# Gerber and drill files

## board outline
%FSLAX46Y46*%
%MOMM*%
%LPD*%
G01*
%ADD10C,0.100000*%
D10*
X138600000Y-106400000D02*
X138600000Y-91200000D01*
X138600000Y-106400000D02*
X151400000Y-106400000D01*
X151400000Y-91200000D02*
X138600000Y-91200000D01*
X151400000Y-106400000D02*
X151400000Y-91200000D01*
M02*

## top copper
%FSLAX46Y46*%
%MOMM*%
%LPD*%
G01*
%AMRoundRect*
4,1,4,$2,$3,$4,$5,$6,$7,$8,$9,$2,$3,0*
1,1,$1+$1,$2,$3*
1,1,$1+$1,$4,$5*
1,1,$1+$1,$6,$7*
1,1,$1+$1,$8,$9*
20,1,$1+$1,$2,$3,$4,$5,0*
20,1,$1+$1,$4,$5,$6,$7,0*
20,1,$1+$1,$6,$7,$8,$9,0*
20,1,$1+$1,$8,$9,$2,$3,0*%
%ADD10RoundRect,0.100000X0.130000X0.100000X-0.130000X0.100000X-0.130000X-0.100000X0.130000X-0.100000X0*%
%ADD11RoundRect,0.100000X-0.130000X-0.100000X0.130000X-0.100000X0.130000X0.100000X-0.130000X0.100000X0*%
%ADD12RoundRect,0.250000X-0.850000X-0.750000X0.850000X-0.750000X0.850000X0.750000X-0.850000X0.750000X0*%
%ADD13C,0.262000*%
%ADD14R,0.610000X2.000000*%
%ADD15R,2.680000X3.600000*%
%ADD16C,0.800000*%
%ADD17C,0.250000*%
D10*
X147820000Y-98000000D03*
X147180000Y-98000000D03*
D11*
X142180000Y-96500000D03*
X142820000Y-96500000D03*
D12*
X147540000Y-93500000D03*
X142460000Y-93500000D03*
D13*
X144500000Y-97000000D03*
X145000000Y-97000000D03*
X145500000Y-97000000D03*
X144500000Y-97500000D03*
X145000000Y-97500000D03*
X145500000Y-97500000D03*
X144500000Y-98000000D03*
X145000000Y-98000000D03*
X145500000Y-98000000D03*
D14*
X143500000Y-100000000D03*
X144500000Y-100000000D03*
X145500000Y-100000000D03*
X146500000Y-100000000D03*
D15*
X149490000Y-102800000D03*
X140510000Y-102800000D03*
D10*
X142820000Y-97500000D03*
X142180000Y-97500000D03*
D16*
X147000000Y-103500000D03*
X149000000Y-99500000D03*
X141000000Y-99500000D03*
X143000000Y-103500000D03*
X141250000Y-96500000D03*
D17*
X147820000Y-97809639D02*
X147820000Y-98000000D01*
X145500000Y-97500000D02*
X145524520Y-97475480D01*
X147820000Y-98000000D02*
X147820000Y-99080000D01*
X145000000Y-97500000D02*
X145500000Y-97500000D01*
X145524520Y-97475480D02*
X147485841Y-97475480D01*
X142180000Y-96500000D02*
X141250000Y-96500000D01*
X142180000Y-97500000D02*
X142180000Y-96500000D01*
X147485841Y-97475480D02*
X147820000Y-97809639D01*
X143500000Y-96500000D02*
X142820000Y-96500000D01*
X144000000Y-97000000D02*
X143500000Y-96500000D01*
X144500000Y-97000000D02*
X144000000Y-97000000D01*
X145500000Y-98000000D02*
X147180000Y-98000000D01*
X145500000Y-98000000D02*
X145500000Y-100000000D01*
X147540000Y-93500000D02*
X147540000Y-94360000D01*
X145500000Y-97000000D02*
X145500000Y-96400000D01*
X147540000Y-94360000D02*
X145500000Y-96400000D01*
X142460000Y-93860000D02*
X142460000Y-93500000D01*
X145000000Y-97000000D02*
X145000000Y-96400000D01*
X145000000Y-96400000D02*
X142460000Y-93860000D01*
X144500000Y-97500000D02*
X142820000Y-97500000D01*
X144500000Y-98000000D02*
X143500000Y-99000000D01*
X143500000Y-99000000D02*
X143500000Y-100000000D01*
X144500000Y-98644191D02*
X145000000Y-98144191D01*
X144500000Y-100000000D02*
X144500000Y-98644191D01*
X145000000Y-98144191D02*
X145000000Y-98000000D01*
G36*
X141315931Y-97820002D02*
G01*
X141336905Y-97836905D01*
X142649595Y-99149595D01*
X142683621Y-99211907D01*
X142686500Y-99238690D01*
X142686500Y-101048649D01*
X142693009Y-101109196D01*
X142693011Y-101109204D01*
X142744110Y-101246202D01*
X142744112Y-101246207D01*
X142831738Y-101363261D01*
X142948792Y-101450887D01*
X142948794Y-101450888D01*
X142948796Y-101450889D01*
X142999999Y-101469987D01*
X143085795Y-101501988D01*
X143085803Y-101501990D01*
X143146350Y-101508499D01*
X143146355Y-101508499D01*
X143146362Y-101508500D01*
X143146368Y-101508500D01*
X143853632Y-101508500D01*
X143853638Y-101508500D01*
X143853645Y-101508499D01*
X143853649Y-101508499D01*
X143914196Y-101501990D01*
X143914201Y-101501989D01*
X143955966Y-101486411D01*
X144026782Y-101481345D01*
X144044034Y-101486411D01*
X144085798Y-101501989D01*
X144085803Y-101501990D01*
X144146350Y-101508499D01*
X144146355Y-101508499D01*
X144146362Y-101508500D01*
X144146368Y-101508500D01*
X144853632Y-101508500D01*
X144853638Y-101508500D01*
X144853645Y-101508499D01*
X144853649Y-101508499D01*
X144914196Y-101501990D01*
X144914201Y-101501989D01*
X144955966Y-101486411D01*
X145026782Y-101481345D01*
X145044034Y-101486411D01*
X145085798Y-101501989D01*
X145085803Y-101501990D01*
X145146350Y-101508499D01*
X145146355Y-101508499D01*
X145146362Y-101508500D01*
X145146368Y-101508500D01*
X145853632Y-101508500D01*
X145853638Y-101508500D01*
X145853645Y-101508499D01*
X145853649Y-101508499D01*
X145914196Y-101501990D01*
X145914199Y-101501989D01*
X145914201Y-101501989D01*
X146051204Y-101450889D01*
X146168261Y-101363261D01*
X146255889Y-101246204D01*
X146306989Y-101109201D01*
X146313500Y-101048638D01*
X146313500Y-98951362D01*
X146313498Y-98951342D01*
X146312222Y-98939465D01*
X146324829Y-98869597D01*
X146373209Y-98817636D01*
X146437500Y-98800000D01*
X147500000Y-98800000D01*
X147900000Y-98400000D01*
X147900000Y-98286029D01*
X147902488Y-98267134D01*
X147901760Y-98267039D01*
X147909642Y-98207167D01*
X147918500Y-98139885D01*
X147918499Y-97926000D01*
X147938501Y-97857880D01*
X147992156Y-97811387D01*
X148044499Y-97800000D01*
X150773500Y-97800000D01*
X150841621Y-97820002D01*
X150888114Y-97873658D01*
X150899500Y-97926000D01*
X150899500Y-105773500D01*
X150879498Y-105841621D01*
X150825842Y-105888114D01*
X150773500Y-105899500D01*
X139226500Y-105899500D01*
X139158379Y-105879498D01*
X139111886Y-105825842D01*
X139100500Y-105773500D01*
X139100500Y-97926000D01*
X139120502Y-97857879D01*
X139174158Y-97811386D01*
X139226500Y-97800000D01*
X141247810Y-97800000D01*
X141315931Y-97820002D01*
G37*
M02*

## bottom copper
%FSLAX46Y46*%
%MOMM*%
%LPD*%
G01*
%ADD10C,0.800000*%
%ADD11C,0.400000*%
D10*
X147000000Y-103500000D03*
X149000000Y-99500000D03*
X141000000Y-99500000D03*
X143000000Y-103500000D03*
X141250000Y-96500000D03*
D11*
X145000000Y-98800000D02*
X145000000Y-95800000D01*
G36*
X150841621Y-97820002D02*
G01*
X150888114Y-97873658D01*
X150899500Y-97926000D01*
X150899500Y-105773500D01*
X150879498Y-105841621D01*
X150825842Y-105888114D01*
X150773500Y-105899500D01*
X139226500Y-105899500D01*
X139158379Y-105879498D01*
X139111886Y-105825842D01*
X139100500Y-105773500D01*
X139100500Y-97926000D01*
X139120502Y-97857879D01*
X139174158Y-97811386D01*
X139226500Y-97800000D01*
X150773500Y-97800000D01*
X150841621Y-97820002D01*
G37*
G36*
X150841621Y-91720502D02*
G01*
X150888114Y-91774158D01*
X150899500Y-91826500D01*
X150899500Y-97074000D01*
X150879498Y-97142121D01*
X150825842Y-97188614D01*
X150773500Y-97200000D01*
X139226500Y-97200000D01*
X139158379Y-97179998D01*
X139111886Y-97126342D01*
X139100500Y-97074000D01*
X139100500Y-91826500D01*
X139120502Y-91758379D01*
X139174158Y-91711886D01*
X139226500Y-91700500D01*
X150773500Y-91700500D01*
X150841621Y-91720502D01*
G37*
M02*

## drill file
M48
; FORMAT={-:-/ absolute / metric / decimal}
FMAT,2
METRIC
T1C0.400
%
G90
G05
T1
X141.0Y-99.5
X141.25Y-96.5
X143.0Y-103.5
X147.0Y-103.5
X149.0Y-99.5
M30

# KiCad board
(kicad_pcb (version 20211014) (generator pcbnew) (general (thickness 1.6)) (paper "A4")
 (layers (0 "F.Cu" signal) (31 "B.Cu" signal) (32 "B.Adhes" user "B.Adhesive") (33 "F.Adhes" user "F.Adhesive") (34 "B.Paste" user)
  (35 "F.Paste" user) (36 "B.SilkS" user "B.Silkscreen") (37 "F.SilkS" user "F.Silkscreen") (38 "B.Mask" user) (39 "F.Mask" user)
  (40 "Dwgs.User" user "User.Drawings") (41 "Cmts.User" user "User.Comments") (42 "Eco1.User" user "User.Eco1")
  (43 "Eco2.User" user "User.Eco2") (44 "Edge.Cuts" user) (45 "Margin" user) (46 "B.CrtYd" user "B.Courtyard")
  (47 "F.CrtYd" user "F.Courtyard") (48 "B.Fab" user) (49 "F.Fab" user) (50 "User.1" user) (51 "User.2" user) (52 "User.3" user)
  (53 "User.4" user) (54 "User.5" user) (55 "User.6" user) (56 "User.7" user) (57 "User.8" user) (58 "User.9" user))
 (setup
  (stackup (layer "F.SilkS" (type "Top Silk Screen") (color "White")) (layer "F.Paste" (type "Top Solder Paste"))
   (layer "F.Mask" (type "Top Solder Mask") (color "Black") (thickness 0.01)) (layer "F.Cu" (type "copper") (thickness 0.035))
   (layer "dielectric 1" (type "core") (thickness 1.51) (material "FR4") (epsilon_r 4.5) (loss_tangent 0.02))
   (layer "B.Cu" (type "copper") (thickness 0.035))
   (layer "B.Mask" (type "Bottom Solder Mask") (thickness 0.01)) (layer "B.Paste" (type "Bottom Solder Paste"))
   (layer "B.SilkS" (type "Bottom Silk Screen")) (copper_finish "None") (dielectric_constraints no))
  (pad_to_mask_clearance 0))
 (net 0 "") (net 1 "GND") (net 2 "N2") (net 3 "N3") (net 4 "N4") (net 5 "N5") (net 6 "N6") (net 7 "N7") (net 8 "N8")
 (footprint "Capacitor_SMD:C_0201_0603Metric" (layer "F.Cu") (at 147.5 98 180)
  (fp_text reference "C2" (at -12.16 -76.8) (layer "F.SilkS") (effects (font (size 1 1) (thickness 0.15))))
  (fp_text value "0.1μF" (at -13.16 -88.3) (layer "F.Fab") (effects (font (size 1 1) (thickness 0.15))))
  (pad "" smd roundrect (at -0.345 0 180) (size 0.318 0.36) (layers "F.Paste") (roundrect_rratio 0.25))
  (pad "" smd roundrect (at 0.345 0 180) (size 0.318 0.36) (layers "F.Paste") (roundrect_rratio 0.25))
  (pad "1" smd roundrect (at -0.32 0 180) (size 0.46 0.4) (layers "F.Cu" "F.Mask") (roundrect_rratio 0.25) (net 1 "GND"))
  (pad "2" smd roundrect (at 0.32 0 180) (size 0.46 0.4) (layers "F.Cu" "F.Mask") (roundrect_rratio 0.25) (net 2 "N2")))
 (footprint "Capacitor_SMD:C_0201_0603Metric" (layer "F.Cu") (at 142.5 96.5)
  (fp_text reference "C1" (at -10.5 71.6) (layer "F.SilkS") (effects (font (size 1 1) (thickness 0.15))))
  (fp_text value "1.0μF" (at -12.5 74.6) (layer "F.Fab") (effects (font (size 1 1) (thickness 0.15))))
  (pad "" smd roundrect (at 0.345 0) (size 0.318 0.36) (layers "F.Paste") (roundrect_rratio 0.25))
  (pad "" smd roundrect (at -0.345 0) (size 0.318 0.36) (layers "F.Paste") (roundrect_rratio 0.25))
  (pad "1" smd roundrect (at -0.32 0) (size 0.46 0.4) (layers "F.Cu" "F.Mask") (roundrect_rratio 0.25) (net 1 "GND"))
  (pad "2" smd roundrect (at 0.32 0) (size 0.46 0.4) (layers "F.Cu" "F.Mask") (roundrect_rratio 0.25) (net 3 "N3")))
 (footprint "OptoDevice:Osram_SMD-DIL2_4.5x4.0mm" (layer "F.Cu") (at 145 93.5 180)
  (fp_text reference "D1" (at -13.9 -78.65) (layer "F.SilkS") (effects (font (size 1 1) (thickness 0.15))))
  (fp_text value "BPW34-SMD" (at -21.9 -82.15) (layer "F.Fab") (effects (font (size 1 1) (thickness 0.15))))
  (pad "1" smd roundrect (at -2.54 0) (size 2.2 2) (layers "F.Cu" "F.Paste" "F.Mask") (roundrect_rratio 0.125) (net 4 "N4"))
  (pad "2" smd roundrect (at 2.54 0) (size 2.2 2) (layers "F.Cu" "F.Paste" "F.Mask") (roundrect_rratio 0.125) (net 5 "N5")))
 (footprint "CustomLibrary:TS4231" (layer "F.Cu") (at 145 97.5)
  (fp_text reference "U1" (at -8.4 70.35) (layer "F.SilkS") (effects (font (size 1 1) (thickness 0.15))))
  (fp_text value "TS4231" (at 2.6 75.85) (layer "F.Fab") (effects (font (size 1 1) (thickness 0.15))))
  (pad "1" smd circle locked (at -0.5 -0.5) (size 0.262 0.262) (layers "F.Cu" "F.Paste" "F.Mask") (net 3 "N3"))
  (pad "2" smd circle locked (at 0 -0.5) (size 0.262 0.262) (layers "F.Cu" "F.Paste" "F.Mask") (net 5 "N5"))
  (pad "3" smd circle locked (at 0.5 -0.5) (size 0.262 0.262) (layers "F.Cu" "F.Paste" "F.Mask") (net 4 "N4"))
  (pad "4" smd circle locked (at -0.5 0) (size 0.262 0.262) (layers "F.Cu" "F.Paste" "F.Mask") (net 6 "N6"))
  (pad "5" smd circle locked (at 0 0) (size 0.262 0.262) (layers "F.Cu" "F.Paste" "F.Mask") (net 1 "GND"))
  (pad "6" smd circle locked (at 0.5 0) (size 0.262 0.262) (layers "F.Cu" "F.Paste" "F.Mask") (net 1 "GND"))
  (pad "7" smd circle locked (at -0.5 0.5) (size 0.262 0.262) (layers "F.Cu" "F.Paste" "F.Mask") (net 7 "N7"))
  (pad "8" smd circle locked (at 0 0.5) (size 0.262 0.262) (layers "F.Cu" "F.Paste" "F.Mask") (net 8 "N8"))
  (pad "9" smd circle locked (at 0.5 0.5) (size 0.262 0.262) (layers "F.Cu" "F.Paste" "F.Mask") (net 2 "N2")))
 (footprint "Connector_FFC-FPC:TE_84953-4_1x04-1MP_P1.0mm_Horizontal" (layer "F.Cu") (at 145 101.8)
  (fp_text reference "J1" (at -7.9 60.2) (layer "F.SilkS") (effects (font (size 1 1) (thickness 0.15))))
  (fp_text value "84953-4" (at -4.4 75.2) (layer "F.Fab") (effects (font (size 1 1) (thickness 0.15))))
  (pad "1" smd rect (at -1.5 -1.8) (size 0.61 2) (layers "F.Cu" "F.Paste" "F.Mask") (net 7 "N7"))
  (pad "2" smd rect (at -0.5 -1.8) (size 0.61 2) (layers "F.Cu" "F.Paste" "F.Mask") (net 8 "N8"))
  (pad "3" smd rect (at 0.5 -1.8) (size 0.61 2) (layers "F.Cu" "F.Paste" "F.Mask") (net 2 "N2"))
  (pad "4" smd rect (at 1.5 -1.8) (size 0.61 2) (layers "F.Cu" "F.Paste" "F.Mask") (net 1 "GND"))
  (pad "MP" smd rect (at 4.49 1) (size 2.68 3.6) (layers "F.Cu" "F.Paste" "F.Mask") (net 1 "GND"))
  (pad "MP" smd rect (at -4.49 1) (size 2.68 3.6) (layers "F.Cu" "F.Paste" "F.Mask") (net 1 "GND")))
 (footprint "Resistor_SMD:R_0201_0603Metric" (layer "F.Cu") (at 142.5 97.5 180)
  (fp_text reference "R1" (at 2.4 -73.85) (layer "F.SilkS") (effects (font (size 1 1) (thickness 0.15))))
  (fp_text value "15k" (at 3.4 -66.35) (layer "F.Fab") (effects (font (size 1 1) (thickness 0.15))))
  (pad "" smd roundrect (at -0.345 0 180) (size 0.318 0.36) (layers "F.Paste") (roundrect_rratio 0.25))
  (pad "" smd roundrect (at 0.345 0 180) (size 0.318 0.36) (layers "F.Paste") (roundrect_rratio 0.25))
  (pad "1" smd roundrect (at -0.32 0 180) (size 0.46 0.4) (layers "F.Cu" "F.Mask") (roundrect_rratio 0.25) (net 6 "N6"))
  (pad "2" smd roundrect (at 0.32 0 180) (size 0.46 0.4) (layers "F.Cu" "F.Mask") (roundrect_rratio 0.25) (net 1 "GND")))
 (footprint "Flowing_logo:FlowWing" (layer "F.Cu") (at 149.7 97.4 90)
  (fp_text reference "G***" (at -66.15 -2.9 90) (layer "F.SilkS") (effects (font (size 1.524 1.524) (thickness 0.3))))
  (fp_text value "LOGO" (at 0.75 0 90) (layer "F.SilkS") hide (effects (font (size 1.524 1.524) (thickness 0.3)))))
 (gr_line (start 138.6 106.4) (end 138.6 91.2) (layer "Edge.Cuts") (width 0.1))
 (gr_line (start 138.6 106.4) (end 151.4 106.4) (layer "Edge.Cuts") (width 0.1))
 (gr_line (start 151.4 91.2) (end 138.6 91.2) (layer "Edge.Cuts") (width 0.1))
 (gr_line (start 151.4 106.4) (end 151.4 91.2) (layer "Edge.Cuts") (width 0.1))
 (segment (start 147.82 97.809639) (end 147.82 98) (width 0.25) (layer "F.Cu") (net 1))
 (segment (start 145.5 97.5) (end 145.52452 97.47548) (width 0.25) (layer "F.Cu") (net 1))
 (segment (start 147.82 98) (end 147.82 99.08) (width 0.25) (layer "F.Cu") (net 1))
 (segment (start 145 97.5) (end 145.5 97.5) (width 0.25) (layer "F.Cu") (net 1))
 (segment (start 145.52452 97.47548) (end 147.485841 97.47548) (width 0.25) (layer "F.Cu") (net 1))
 (segment (start 142.18 96.5) (end 141.25 96.5) (width 0.25) (layer "F.Cu") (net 1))
 (segment (start 142.18 97.5) (end 142.18 96.5) (width 0.25) (layer "F.Cu") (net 1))
 (segment (start 147.485841 97.47548) (end 147.82 97.809639) (width 0.25) (layer "F.Cu") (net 1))
 (via (at 147 103.5) (size 0.8) (drill 0.4) (layers "F.Cu" "B.Cu") (free) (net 1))
 (via (at 149 99.5) (size 0.8) (drill 0.4) (layers "F.Cu" "B.Cu") (free) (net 1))
 (via (at 141 99.5) (size 0.8) (drill 0.4) (layers "F.Cu" "B.Cu") (free) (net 1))
 (via (at 143 103.5) (size 0.8) (drill 0.4) (layers "F.Cu" "B.Cu") (free) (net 1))
 (via (at 141.25 96.5) (size 0.8) (drill 0.4) (layers "F.Cu" "B.Cu") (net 1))
 (segment (start 145 98.8) (end 145 95.8) (width 0.4) (layer "B.Cu") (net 1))
 (segment (start 143.5 96.5) (end 142.82 96.5) (width 0.25) (layer "F.Cu") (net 3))
 (segment (start 144 97) (end 143.5 96.5) (width 0.25) (layer "F.Cu") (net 3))
 (segment (start 144.5 97) (end 144 97) (width 0.25) (layer "F.Cu") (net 3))
 (segment (start 145.5 98) (end 147.18 98) (width 0.25) (layer "F.Cu") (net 2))
 (segment (start 145.5 98) (end 145.5 100) (width 0.25) (layer "F.Cu") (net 2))
 (segment (start 147.54 93.5) (end 147.54 94.36) (width 0.25) (layer "F.Cu") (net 4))
 (segment (start 145.5 97) (end 145.5 96.4) (width 0.25) (layer "F.Cu") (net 4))
 (segment (start 147.54 94.36) (end 145.5 96.4) (width 0.25) (layer "F.Cu") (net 4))
 (segment (start 142.46 93.86) (end 142.46 93.5) (width 0.25) (layer "F.Cu") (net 5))
 (segment (start 145 97) (end 145 96.4) (width 0.25) (layer "F.Cu") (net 5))
 (segment (start 145 96.4) (end 142.46 93.86) (width 0.25) (layer "F.Cu") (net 5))
 (segment (start 144.5 97.5) (end 142.82 97.5) (width 0.25) (layer "F.Cu") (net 6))
 (segment (start 144.5 98) (end 143.5 99) (width 0.25) (layer "F.Cu") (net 7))
 (segment (start 143.5 99) (end 143.5 100) (width 0.25) (layer "F.Cu") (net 7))
 (segment (start 144.5 98.644191) (end 145 98.144191) (width 0.25) (layer "F.Cu") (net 8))
 (segment (start 144.5 100) (end 144.5 98.644191) (width 0.25) (layer "F.Cu") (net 8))
 (segment (start 145 98.144191) (end 145 98) (width 0.25) (layer "F.Cu") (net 8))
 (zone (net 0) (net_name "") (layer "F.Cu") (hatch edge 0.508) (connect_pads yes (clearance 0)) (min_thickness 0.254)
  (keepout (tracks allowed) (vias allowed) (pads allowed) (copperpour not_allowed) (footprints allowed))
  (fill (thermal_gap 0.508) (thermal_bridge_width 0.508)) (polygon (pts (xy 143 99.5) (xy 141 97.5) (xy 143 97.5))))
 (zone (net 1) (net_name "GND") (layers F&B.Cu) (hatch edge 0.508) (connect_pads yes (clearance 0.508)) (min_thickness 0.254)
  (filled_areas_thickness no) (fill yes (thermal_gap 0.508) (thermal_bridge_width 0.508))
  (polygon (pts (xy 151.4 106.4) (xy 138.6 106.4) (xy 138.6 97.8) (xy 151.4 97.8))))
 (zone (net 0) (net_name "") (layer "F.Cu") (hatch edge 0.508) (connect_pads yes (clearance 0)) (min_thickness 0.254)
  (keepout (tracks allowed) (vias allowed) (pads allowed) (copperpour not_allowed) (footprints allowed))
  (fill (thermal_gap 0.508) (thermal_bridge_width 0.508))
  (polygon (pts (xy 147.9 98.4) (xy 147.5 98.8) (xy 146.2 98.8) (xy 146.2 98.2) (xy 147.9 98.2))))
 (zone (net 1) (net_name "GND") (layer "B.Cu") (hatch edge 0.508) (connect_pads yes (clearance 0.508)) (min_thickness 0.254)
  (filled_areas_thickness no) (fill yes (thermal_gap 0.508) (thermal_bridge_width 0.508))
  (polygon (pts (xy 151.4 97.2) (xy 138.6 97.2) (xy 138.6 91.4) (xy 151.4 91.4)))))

